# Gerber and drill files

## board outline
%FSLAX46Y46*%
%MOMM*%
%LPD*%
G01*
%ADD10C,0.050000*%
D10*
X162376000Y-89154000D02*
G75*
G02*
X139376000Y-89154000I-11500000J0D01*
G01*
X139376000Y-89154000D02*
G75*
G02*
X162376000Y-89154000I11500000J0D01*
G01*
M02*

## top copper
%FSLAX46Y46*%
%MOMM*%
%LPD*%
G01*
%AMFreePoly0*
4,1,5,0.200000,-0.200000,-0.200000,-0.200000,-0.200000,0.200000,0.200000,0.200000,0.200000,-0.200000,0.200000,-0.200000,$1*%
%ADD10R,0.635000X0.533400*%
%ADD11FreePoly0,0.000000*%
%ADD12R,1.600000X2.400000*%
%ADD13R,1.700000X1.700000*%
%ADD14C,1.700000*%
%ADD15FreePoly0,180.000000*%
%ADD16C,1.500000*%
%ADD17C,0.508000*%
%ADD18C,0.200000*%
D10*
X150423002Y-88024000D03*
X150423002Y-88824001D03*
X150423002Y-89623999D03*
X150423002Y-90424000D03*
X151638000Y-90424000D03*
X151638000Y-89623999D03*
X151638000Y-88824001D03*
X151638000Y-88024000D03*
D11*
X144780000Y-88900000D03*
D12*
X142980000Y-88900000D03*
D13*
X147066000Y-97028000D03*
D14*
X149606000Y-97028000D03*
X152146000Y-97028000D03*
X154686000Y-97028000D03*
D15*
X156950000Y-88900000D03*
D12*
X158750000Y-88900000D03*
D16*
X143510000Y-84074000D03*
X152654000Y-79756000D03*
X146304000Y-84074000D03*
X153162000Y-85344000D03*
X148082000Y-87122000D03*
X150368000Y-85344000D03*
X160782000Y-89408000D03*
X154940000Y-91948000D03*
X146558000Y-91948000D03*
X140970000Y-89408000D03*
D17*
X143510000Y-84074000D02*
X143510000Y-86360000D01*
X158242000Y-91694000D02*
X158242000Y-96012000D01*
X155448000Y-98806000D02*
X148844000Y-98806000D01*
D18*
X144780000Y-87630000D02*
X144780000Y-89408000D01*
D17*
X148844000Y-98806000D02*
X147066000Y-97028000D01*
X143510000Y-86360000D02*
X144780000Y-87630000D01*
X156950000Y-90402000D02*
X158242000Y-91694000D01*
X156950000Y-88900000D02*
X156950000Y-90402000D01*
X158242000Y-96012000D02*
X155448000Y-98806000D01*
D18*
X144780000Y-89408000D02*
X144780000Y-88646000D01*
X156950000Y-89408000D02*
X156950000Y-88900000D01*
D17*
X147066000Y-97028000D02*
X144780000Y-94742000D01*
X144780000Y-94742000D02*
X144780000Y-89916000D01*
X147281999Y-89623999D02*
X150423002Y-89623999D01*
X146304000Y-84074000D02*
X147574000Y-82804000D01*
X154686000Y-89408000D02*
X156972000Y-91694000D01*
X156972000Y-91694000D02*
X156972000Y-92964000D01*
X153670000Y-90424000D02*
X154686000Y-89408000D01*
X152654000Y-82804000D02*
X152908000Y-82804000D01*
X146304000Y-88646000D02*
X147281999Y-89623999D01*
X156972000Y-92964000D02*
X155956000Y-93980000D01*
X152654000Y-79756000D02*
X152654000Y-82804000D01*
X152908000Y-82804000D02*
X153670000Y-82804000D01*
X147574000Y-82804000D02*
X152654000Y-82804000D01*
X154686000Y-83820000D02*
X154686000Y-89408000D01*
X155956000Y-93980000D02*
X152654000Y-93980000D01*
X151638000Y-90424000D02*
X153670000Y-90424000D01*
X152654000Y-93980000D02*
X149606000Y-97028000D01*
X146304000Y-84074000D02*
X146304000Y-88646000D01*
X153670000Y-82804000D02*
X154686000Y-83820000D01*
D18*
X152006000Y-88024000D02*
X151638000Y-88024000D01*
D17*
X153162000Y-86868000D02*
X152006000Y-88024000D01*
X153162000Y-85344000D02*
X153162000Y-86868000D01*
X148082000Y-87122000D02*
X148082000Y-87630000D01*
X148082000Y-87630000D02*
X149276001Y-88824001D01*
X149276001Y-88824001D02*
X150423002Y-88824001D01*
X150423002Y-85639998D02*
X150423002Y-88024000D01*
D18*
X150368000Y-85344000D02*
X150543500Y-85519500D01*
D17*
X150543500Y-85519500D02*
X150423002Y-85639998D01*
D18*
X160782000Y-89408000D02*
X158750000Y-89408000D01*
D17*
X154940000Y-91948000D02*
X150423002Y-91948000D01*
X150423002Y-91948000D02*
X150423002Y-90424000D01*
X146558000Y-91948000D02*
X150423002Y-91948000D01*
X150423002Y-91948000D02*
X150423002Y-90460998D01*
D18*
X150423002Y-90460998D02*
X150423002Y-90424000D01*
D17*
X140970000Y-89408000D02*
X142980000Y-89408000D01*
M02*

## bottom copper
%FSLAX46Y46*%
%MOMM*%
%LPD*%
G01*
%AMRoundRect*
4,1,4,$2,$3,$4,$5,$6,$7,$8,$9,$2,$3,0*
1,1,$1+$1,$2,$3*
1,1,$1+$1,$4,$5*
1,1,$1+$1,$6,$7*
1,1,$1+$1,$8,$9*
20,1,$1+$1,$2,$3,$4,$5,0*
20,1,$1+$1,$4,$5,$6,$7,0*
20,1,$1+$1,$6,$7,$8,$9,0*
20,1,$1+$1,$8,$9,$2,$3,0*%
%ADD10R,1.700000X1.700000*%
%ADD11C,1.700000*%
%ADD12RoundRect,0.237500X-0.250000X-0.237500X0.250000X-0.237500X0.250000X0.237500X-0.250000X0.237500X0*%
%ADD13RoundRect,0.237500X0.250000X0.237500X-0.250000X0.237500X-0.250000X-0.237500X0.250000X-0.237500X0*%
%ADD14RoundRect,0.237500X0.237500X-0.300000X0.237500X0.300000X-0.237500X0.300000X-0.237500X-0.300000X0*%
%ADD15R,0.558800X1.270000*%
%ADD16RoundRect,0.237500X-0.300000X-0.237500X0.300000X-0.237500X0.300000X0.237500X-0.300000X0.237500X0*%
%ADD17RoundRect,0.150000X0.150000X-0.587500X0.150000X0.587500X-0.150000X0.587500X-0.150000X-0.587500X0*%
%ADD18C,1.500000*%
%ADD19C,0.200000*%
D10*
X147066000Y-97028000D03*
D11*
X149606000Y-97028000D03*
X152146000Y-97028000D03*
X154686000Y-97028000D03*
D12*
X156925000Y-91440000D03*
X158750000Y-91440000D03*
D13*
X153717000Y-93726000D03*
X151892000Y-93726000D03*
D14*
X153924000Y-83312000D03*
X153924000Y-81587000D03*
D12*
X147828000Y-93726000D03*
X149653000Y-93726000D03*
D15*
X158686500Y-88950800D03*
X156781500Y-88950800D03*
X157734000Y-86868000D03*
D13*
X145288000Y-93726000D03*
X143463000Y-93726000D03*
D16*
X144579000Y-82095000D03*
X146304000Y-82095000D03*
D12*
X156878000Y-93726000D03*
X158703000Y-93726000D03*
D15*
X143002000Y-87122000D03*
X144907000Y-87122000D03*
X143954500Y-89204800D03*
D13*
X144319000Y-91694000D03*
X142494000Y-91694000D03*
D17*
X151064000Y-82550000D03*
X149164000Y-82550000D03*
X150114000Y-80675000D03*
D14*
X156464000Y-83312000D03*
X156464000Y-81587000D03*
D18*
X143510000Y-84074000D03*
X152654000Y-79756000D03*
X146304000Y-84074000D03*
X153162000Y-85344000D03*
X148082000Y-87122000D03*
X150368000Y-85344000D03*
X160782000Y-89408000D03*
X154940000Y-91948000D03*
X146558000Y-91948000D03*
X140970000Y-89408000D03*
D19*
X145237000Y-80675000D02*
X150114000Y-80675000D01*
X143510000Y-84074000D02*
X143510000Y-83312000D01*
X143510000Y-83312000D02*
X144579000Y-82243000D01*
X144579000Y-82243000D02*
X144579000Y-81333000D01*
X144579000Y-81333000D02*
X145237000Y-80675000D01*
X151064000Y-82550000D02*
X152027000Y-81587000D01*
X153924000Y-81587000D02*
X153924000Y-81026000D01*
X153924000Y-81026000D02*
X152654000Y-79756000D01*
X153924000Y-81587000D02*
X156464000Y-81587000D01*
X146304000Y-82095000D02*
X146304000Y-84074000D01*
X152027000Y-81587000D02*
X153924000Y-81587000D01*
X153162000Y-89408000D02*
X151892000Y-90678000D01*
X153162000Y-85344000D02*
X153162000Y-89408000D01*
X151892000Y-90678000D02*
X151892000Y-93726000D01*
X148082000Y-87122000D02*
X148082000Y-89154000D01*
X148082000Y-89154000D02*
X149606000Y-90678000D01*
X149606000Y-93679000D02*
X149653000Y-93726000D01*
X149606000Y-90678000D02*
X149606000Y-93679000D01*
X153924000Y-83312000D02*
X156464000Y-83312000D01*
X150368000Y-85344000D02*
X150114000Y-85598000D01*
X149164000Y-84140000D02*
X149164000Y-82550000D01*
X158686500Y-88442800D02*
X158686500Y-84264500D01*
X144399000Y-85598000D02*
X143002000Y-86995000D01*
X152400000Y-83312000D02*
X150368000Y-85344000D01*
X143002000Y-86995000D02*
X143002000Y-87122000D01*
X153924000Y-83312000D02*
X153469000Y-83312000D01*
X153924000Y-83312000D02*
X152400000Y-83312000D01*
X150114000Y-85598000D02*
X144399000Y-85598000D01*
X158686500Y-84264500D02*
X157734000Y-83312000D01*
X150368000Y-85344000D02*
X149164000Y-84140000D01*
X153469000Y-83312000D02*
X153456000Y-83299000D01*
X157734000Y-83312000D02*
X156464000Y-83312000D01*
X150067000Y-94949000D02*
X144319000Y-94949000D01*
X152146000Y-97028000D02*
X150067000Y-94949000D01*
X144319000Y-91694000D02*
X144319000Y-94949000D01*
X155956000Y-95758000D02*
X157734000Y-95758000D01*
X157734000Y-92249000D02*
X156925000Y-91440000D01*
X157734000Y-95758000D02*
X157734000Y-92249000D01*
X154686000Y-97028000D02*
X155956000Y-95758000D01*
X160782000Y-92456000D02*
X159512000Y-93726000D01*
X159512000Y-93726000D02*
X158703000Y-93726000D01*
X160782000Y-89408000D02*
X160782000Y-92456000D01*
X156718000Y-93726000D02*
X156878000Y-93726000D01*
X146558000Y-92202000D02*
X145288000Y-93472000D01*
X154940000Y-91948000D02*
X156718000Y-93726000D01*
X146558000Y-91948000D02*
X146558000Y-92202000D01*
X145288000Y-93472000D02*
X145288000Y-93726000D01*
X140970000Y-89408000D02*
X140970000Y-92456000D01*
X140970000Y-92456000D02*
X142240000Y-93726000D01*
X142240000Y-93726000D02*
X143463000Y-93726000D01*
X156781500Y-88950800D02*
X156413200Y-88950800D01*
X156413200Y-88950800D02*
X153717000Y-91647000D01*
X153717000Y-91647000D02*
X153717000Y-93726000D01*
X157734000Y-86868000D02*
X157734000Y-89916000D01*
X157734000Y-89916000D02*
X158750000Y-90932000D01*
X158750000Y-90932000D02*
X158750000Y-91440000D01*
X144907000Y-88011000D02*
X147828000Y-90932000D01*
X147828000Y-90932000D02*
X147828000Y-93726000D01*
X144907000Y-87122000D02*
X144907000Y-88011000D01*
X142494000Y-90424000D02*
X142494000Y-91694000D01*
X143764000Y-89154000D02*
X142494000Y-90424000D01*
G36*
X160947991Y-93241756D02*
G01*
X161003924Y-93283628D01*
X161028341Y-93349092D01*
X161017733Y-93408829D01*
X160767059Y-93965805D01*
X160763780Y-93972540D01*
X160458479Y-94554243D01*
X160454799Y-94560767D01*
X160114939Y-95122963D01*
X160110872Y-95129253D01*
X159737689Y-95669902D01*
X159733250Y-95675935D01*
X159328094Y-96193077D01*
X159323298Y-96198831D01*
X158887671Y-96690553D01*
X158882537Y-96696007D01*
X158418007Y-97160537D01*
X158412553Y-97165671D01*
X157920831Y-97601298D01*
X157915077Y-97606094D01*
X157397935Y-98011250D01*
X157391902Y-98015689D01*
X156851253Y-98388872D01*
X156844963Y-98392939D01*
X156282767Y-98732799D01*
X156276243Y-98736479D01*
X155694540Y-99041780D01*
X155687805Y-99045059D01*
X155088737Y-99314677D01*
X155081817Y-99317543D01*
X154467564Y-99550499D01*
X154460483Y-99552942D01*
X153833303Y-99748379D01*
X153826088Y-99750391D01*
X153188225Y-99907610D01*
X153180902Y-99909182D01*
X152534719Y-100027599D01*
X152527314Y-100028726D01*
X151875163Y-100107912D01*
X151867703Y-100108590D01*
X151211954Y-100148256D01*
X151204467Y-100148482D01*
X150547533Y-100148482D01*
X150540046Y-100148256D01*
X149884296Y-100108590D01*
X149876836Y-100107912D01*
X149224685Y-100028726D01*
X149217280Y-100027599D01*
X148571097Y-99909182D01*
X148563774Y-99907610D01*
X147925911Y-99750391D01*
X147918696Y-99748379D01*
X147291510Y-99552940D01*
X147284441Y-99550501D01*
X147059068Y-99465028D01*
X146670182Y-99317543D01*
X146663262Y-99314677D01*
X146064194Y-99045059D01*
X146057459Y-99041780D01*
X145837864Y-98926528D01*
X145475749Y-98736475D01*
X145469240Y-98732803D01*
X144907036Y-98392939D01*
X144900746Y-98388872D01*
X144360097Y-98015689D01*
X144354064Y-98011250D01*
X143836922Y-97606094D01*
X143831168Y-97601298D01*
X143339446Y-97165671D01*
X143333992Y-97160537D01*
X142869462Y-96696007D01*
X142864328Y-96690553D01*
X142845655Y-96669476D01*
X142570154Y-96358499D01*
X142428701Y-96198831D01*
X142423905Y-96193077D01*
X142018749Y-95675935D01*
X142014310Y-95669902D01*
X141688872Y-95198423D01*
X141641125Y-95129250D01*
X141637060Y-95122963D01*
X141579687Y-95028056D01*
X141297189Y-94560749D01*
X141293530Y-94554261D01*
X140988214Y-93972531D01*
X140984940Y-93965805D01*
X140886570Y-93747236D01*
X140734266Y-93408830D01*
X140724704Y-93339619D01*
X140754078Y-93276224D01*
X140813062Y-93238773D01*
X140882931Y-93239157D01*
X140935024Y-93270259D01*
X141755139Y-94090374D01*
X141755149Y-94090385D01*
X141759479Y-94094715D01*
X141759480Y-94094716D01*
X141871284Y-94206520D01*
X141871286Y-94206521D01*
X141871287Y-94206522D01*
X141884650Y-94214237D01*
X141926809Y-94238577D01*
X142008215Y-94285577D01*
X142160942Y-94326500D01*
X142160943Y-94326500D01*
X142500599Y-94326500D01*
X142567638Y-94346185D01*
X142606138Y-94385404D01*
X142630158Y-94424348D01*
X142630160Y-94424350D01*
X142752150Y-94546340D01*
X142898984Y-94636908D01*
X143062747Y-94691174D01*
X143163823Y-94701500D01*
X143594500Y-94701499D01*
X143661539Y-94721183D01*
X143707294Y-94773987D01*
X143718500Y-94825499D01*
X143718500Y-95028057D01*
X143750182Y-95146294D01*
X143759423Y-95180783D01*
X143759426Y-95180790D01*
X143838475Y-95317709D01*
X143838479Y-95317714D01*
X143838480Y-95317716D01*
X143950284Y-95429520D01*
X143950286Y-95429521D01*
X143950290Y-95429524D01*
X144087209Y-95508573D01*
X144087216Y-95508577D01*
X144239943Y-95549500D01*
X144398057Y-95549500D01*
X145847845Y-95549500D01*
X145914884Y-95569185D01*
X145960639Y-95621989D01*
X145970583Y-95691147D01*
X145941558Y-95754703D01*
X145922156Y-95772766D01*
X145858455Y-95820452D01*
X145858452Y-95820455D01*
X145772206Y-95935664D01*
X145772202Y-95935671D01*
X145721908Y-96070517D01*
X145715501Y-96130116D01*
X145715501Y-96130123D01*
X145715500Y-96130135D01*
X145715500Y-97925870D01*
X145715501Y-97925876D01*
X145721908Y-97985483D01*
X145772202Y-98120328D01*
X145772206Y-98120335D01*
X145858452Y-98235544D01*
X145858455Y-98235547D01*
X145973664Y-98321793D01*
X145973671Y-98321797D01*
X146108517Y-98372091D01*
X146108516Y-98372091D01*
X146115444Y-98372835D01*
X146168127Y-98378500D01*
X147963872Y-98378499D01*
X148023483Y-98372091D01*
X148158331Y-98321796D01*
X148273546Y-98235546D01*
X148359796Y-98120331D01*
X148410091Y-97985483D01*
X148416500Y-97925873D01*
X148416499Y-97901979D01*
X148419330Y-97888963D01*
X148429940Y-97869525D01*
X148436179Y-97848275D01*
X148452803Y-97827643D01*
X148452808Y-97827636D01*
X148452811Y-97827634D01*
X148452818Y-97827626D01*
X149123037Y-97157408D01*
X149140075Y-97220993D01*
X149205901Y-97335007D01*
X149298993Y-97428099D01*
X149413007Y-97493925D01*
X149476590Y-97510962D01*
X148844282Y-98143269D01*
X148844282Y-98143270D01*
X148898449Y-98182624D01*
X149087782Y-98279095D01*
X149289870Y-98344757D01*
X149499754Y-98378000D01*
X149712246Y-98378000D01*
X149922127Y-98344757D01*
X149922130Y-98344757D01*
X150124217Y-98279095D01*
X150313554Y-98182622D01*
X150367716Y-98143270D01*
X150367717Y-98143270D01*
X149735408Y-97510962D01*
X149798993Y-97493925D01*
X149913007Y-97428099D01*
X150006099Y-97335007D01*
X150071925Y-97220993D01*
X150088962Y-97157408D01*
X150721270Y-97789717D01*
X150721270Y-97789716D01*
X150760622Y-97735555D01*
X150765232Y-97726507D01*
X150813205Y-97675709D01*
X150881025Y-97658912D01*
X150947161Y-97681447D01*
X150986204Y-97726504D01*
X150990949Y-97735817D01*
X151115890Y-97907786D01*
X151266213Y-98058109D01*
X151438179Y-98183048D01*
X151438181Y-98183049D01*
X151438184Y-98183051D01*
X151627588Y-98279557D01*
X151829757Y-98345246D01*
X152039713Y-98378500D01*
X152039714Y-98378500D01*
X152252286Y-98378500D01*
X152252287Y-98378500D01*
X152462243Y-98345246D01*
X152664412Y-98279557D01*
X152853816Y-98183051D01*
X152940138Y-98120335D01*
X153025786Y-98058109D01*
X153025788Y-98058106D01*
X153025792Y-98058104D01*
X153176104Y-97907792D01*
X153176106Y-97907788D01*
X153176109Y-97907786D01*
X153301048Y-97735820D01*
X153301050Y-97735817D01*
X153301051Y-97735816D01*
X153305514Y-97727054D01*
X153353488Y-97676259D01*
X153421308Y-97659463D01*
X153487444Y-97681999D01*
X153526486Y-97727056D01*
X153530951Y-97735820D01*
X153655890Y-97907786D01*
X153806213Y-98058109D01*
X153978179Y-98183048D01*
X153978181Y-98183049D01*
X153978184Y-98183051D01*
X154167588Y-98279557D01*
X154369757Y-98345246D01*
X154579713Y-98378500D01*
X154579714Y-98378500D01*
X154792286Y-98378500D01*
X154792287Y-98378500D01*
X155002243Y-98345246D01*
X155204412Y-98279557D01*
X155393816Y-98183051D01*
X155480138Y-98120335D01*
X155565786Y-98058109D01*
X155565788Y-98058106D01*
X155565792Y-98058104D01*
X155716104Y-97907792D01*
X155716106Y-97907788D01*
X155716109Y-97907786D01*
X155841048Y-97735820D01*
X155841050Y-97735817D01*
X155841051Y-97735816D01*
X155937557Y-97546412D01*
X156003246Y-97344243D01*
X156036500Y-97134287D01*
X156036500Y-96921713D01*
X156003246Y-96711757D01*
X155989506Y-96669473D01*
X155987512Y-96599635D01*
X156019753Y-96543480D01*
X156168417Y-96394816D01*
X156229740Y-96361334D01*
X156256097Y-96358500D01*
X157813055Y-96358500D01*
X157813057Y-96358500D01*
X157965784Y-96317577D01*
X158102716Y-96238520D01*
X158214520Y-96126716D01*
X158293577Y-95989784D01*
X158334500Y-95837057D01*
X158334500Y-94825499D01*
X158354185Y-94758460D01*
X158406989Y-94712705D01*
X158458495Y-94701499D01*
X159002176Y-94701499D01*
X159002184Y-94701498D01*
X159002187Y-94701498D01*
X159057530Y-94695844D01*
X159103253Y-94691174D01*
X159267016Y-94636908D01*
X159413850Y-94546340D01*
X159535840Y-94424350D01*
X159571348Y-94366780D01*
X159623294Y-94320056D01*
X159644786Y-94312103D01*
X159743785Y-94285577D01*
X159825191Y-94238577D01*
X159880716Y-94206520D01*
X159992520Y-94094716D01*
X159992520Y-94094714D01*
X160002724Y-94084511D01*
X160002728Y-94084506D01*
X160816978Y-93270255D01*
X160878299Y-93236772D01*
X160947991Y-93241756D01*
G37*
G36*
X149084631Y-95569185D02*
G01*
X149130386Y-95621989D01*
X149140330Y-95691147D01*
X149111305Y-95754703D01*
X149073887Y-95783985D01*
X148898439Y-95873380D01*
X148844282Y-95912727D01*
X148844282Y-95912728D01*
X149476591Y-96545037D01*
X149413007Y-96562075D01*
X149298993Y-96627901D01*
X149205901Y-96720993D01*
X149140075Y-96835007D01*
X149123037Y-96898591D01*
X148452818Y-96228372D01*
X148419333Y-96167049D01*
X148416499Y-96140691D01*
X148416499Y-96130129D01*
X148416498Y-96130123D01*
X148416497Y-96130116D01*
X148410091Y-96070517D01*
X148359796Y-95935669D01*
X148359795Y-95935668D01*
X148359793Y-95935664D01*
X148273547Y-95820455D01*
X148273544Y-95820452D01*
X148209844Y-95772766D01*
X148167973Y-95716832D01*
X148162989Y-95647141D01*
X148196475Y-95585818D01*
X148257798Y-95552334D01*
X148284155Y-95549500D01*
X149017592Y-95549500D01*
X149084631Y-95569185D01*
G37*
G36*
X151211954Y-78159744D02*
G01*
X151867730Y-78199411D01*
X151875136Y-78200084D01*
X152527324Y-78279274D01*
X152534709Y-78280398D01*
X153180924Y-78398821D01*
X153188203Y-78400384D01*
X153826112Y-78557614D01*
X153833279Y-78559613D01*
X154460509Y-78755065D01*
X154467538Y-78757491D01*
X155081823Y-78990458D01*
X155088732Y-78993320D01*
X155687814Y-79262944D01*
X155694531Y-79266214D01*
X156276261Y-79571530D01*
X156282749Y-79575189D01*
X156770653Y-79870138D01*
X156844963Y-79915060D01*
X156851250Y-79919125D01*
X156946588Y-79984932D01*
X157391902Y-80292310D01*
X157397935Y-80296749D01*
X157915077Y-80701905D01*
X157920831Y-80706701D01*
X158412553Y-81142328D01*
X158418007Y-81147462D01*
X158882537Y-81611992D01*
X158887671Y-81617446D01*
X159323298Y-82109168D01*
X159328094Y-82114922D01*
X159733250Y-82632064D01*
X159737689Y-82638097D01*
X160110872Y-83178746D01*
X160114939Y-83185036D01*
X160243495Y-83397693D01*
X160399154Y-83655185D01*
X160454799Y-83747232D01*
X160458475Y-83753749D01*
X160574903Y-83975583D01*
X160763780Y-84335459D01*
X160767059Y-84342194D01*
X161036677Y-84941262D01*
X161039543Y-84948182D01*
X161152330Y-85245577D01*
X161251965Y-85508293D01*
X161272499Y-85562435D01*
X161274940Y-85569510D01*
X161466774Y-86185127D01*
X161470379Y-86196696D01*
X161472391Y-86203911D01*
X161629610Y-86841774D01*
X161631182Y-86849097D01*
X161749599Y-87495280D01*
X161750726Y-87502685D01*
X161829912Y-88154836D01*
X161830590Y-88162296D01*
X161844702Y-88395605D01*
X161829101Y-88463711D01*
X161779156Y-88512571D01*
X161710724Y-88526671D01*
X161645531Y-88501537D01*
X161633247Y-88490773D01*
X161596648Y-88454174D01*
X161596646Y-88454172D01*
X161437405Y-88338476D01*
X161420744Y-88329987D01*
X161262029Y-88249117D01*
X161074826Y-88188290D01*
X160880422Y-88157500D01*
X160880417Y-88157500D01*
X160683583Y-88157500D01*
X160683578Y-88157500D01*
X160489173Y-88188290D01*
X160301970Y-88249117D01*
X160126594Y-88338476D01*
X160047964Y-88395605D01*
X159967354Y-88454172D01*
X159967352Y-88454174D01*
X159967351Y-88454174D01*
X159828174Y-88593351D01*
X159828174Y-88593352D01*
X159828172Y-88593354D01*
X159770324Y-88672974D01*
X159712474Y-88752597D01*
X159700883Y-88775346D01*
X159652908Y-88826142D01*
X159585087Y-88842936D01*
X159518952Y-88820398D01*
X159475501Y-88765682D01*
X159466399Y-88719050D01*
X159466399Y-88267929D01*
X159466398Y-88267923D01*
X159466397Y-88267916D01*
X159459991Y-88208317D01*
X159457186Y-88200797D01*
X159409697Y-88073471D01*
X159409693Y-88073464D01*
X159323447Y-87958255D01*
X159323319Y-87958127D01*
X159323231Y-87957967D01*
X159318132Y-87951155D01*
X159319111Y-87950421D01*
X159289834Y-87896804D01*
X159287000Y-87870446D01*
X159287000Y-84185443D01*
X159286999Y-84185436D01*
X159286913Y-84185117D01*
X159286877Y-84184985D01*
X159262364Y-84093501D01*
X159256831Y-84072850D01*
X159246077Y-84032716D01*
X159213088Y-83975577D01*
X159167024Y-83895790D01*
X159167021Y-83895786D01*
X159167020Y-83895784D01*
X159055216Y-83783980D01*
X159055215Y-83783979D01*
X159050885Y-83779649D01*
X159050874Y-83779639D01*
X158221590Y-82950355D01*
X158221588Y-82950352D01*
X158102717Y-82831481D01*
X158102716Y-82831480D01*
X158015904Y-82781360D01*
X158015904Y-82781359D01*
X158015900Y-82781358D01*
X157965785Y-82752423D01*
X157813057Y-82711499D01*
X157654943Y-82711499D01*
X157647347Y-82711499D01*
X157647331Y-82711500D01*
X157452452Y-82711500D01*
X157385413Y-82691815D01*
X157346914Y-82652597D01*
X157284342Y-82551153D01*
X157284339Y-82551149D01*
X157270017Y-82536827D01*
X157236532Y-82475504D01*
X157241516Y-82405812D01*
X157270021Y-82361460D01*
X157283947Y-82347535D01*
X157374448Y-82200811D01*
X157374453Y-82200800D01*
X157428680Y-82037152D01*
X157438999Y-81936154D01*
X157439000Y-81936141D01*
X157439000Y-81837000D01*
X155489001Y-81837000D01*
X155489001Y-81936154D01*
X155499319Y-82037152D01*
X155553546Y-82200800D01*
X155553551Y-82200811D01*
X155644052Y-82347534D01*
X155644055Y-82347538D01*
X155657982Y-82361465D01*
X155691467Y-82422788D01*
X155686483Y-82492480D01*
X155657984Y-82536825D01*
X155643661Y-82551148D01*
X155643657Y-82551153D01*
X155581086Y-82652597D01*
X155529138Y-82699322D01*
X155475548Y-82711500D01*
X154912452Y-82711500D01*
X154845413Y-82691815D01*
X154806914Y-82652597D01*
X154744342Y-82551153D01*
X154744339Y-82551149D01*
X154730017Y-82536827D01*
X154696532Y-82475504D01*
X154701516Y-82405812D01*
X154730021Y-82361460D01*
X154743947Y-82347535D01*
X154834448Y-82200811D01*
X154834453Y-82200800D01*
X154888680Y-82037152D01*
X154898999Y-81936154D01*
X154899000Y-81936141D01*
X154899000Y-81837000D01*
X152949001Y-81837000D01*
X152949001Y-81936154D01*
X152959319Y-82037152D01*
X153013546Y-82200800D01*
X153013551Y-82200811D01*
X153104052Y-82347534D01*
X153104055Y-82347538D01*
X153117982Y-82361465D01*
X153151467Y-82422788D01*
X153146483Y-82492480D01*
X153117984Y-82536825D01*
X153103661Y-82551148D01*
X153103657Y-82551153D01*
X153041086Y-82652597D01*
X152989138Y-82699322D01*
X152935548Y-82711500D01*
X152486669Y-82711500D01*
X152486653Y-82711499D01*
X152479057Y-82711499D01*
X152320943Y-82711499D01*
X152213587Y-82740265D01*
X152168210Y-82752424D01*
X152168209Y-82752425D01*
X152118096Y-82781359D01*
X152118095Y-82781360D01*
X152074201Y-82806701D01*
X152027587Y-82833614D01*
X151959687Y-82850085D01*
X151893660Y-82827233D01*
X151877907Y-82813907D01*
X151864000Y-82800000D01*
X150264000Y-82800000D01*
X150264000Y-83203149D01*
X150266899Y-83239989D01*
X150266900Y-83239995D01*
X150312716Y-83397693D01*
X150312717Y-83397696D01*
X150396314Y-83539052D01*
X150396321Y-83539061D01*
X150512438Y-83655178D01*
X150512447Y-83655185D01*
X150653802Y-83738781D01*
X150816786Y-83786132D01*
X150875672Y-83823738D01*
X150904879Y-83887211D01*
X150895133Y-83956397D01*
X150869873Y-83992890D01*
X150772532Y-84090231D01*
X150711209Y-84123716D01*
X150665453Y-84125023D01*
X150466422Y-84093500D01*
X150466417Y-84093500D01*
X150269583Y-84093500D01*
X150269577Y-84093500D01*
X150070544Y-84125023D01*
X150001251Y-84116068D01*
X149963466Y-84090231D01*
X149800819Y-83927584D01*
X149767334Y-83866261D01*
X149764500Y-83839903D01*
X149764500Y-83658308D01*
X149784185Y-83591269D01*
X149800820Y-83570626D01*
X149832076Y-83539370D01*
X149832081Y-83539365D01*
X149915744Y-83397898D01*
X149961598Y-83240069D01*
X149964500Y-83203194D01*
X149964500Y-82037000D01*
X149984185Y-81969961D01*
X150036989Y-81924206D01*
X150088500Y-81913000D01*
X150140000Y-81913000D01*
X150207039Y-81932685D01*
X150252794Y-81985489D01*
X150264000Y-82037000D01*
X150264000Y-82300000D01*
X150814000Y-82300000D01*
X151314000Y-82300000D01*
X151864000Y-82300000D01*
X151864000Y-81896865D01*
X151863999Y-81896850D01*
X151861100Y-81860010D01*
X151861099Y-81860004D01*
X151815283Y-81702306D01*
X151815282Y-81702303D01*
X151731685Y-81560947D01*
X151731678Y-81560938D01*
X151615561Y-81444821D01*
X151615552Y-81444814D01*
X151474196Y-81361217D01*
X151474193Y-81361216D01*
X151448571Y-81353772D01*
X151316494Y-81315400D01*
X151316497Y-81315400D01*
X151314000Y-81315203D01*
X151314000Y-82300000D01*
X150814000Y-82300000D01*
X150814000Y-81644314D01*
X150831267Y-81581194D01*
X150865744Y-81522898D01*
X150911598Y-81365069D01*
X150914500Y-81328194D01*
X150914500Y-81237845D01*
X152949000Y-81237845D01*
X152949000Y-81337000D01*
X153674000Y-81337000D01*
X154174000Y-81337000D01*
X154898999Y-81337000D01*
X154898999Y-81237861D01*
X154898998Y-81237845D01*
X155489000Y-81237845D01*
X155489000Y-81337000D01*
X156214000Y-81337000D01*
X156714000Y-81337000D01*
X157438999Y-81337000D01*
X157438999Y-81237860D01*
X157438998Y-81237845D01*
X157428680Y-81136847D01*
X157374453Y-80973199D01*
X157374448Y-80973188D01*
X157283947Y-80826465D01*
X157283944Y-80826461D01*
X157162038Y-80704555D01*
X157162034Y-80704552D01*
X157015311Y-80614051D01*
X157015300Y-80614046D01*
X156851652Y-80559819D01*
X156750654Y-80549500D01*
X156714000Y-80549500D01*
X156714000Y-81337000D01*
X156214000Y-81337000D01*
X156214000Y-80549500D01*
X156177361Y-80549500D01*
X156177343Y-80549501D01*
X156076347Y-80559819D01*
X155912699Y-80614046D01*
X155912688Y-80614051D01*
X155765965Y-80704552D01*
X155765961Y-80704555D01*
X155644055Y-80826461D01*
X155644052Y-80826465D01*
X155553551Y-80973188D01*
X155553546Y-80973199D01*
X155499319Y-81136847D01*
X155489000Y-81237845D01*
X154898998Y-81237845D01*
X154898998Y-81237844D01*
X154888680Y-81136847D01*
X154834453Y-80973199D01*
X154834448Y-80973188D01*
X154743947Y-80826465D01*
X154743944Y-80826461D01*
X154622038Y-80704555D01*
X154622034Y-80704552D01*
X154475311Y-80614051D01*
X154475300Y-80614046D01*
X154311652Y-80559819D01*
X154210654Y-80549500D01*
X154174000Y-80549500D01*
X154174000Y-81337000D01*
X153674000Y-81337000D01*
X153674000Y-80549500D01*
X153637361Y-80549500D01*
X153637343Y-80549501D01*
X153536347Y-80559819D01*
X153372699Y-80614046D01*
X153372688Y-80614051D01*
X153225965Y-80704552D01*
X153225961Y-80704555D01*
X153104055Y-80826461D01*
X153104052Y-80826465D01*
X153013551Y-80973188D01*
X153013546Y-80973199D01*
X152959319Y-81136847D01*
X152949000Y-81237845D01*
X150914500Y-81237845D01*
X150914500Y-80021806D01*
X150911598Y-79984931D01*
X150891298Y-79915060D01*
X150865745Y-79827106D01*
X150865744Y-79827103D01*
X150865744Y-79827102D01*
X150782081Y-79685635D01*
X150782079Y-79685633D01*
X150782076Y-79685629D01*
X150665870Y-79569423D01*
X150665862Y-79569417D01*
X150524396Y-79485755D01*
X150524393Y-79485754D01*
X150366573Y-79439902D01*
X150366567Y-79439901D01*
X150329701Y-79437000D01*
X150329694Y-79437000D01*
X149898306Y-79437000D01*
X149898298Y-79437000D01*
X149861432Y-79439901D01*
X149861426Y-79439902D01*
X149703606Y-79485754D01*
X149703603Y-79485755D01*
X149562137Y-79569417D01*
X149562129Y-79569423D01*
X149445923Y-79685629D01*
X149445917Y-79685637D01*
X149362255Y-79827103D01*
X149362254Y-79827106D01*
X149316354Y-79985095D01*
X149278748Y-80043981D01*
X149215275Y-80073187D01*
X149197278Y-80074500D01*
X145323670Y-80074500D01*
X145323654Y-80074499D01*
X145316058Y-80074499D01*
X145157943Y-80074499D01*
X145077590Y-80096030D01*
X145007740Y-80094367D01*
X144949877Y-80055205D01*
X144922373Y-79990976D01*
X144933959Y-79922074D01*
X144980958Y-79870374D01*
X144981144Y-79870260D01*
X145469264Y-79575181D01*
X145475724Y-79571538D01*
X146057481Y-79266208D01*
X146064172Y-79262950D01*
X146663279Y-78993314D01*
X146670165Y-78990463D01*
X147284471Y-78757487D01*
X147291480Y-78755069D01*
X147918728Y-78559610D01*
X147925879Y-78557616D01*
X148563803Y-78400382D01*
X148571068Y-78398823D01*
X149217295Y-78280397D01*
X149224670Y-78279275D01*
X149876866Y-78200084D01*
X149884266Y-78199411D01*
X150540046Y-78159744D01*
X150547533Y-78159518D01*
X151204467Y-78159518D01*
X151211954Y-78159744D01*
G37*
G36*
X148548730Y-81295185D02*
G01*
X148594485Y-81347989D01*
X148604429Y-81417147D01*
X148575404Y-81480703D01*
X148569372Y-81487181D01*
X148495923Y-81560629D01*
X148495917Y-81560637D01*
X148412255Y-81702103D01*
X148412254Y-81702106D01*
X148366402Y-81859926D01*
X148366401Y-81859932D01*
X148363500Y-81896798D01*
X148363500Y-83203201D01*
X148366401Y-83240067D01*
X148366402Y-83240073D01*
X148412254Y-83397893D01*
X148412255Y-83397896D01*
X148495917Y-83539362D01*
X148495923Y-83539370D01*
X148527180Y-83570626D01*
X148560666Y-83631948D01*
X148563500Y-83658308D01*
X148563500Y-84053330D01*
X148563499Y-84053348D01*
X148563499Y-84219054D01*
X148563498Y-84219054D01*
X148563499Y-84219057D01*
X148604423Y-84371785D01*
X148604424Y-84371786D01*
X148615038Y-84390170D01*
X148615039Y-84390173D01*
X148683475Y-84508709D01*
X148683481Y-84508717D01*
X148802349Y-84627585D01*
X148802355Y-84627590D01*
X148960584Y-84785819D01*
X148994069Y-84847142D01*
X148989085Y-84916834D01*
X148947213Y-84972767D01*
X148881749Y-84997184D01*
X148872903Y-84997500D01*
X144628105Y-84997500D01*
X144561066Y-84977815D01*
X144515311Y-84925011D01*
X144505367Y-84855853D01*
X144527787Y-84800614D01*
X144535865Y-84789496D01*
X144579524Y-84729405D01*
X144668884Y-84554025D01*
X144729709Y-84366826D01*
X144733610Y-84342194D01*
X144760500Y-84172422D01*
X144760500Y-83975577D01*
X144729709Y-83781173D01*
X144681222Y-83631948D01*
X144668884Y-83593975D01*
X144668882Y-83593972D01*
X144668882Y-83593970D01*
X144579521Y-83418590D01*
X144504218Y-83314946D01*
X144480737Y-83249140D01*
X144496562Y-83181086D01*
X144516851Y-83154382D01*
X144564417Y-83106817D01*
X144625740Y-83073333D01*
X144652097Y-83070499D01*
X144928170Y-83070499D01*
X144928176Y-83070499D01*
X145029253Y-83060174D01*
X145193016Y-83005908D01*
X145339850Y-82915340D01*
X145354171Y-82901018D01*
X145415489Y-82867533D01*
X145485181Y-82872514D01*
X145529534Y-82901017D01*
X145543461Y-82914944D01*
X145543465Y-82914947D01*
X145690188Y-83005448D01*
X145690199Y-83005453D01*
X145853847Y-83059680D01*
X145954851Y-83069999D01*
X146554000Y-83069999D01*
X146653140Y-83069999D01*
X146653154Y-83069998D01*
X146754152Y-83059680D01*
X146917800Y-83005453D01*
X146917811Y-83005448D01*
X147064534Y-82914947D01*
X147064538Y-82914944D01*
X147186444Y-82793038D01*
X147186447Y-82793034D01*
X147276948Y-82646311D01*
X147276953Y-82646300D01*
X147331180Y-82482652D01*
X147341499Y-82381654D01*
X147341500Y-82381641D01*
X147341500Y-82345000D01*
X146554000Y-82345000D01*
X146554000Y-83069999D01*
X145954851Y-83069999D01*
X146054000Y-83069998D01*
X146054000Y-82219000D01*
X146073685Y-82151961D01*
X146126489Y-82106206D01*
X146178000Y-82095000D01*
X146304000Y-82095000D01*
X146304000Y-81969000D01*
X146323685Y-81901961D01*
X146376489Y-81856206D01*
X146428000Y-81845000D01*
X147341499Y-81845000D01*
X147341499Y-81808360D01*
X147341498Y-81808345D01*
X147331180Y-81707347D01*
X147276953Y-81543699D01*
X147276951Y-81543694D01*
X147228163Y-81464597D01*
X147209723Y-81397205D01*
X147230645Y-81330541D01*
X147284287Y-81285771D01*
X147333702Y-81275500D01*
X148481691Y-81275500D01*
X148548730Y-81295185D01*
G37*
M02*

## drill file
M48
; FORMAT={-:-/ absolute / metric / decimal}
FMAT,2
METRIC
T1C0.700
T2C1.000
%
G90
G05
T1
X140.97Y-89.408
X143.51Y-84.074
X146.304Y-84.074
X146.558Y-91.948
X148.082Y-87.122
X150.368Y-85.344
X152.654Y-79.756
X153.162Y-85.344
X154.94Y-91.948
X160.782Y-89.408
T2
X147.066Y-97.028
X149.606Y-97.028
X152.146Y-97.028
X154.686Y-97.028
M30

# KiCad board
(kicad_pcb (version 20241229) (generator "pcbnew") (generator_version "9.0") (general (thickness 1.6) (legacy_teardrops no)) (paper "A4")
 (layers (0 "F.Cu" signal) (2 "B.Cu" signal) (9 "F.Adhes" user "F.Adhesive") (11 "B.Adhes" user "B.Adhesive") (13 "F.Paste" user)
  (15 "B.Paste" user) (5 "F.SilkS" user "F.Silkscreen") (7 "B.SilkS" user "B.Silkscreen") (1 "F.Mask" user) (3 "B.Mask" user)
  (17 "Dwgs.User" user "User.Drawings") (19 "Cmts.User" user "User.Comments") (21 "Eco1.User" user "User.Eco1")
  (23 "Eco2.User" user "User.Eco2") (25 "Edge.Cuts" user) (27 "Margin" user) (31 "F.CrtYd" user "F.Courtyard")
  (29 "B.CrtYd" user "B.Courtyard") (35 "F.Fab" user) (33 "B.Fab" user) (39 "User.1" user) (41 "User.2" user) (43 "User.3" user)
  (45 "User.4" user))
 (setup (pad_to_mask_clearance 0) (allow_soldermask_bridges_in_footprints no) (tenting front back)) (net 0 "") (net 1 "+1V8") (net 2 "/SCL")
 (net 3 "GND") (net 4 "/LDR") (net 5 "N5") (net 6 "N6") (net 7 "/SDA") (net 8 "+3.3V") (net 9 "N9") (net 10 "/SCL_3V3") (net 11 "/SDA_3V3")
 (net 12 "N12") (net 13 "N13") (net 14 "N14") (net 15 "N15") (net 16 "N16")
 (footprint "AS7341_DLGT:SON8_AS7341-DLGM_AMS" (layer "F.Cu") (at 151.030501 89.224)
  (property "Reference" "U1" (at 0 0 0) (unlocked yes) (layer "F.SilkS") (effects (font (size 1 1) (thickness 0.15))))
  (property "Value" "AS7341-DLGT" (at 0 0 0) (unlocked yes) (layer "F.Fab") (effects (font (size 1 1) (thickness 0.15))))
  (pad "1" smd rect (at -0.607499 -1.2) (size 0.635 0.5334) (layers "F.Cu" "F.Mask" "F.Paste") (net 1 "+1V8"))
  (pad "2" smd rect (at -0.607499 -0.399999) (size 0.635 0.5334) (layers "F.Cu" "F.Mask" "F.Paste") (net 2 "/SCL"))
  (pad "3" smd rect (at -0.607499 0.399999) (size 0.635 0.5334) (layers "F.Cu" "F.Mask" "F.Paste") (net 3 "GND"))
  (pad "4" smd rect (at -0.607499 1.2) (size 0.635 0.5334) (layers "F.Cu" "F.Mask" "F.Paste") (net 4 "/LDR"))
  (pad "5" smd rect (at 0.607499 1.2) (size 0.635 0.5334) (layers "F.Cu" "F.Mask" "F.Paste") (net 3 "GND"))
  (pad "6" smd rect (at 0.607499 0.399999) (size 0.635 0.5334) (layers "F.Cu" "F.Mask" "F.Paste") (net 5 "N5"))
  (pad "7" smd rect (at 0.607499 -0.399999) (size 0.635 0.5334) (layers "F.Cu" "F.Mask" "F.Paste") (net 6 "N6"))
  (pad "8" smd rect (at 0.607499 -1.2) (size 0.635 0.5334) (layers "F.Cu" "F.Mask" "F.Paste") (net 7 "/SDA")))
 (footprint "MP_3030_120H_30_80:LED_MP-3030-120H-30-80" (layer "F.Cu") (at 143.78 88.9)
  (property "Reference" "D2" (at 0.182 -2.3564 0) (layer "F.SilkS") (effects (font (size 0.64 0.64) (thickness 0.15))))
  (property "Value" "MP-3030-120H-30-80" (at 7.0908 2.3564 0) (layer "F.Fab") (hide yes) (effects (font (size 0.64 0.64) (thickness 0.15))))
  (pad "A" smd custom (at 1 0) (size 0.4 0.4) (layers "F.Cu") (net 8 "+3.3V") (options (clearance outline) (anchor rect)) (primitives))
  (pad "C" smd rect (at -0.8 0) (size 1.6 2.4) (layers "F.Cu" "F.Mask" "F.Paste") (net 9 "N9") (solder_mask_margin 0.102)))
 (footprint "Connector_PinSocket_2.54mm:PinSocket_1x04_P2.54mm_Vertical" (layer "F.Cu") (at 147.066 97.028 90)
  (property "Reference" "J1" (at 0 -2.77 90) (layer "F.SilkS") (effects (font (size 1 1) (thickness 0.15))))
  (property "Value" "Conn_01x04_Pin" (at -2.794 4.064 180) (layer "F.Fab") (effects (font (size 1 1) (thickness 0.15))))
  (pad "1" thru_hole rect (at 0 0 90) (size 1.7 1.7) (drill 1) (layers "*.Cu" "*.Mask") (remove_unused_layers no) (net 8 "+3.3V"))
  (pad "2" thru_hole circle (at 0 2.54 90) (size 1.7 1.7) (drill 1) (layers "*.Cu" "*.Mask") (remove_unused_layers no) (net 3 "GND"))
  (pad "3" thru_hole circle (at 0 5.08 90) (size 1.7 1.7) (drill 1) (layers "*.Cu" "*.Mask") (remove_unused_layers no) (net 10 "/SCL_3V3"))
  (pad "4" thru_hole circle (at 0 7.62 90) (size 1.7 1.7) (drill 1) (layers "*.Cu" "*.Mask") (remove_unused_layers no) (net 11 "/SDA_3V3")))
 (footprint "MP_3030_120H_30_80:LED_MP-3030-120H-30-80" (layer "F.Cu") (at 157.95 88.9 180)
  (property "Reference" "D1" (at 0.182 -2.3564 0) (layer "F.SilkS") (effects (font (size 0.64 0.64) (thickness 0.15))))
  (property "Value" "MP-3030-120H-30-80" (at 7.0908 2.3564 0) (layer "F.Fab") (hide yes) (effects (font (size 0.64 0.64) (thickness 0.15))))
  (pad "A" smd custom (at 1 0 180) (size 0.4 0.4) (layers "F.Cu") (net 8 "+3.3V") (options (clearance outline) (anchor rect)) (primitives))
  (pad "C" smd rect (at -0.8 0 180) (size 1.6 2.4) (layers "F.Cu" "F.Mask" "F.Paste") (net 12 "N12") (solder_mask_margin 0.102)))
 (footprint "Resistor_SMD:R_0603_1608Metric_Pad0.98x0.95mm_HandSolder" (layer "B.Cu") (at 157.8375 91.44)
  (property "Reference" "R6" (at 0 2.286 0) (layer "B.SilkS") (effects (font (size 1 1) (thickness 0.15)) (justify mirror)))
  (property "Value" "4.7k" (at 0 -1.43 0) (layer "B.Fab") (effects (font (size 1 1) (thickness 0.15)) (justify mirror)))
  (pad "1" smd roundrect (at -0.9125 0) (size 0.975 0.95) (layers "B.Cu" "B.Mask" "B.Paste") (roundrect_rratio 0.25) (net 11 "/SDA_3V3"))
  (pad "2" smd roundrect (at 0.9125 0) (size 0.975 0.95) (layers "B.Cu" "B.Mask" "B.Paste") (roundrect_rratio 0.25) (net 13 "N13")))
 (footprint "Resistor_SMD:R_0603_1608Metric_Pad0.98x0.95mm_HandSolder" (layer "B.Cu") (at 152.8045 93.726 180)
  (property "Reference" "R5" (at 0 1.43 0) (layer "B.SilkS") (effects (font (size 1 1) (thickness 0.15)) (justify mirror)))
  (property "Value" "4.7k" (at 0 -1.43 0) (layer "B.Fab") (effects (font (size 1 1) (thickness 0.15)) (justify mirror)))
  (pad "1" smd roundrect (at -0.9125 0 180) (size 0.975 0.95) (layers "B.Cu" "B.Mask" "B.Paste") (roundrect_rratio 0.25) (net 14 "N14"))
  (pad "2" smd roundrect (at 0.9125 0 180) (size 0.975 0.95) (layers "B.Cu" "B.Mask" "B.Paste") (roundrect_rratio 0.25) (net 7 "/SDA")))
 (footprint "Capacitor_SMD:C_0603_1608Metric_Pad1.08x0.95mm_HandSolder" (layer "B.Cu") (at 153.924 82.4495 90)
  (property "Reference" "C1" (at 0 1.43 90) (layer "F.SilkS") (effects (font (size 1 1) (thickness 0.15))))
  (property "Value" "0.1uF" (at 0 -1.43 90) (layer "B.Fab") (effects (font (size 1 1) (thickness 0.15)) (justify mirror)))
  (pad "1" smd roundrect (at -0.8625 0 90) (size 1.075 0.95) (layers "B.Cu" "B.Mask" "B.Paste") (roundrect_rratio 0.25) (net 1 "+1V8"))
  (pad "2" smd roundrect (at 0.8625 0 90) (size 1.075 0.95) (layers "B.Cu" "B.Mask" "B.Paste") (roundrect_rratio 0.25) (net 3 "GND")))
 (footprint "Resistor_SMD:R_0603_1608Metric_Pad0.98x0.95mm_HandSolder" (layer "B.Cu") (at 148.7405 93.726)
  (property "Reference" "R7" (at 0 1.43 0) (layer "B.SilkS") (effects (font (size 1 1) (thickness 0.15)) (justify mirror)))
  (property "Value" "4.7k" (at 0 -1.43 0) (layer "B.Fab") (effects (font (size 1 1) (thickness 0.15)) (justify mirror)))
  (pad "1" smd roundrect (at -0.9125 0) (size 0.975 0.95) (layers "B.Cu" "B.Mask" "B.Paste") (roundrect_rratio 0.25) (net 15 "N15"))
  (pad "2" smd roundrect (at 0.9125 0) (size 0.975 0.95) (layers "B.Cu" "B.Mask" "B.Paste") (roundrect_rratio 0.25) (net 2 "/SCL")))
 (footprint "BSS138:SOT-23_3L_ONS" (layer "B.Cu") (at 157.734 87.9094 180)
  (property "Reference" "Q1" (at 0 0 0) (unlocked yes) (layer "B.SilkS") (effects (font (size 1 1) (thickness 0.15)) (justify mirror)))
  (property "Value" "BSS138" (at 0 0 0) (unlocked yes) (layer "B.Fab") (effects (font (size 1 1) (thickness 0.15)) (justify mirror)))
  (pad "1" smd rect (at -0.9525 -1.0414 180) (size 0.5588 1.27) (layers "B.Cu" "B.Mask" "B.Paste") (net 1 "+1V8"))
  (pad "2" smd rect (at 0.9525 -1.0414 180) (size 0.5588 1.27) (layers "B.Cu" "B.Mask" "B.Paste") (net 14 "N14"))
  (pad "3" smd rect (at 0 1.0414 180) (size 0.5588 1.27) (layers "B.Cu" "B.Mask" "B.Paste") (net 13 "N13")))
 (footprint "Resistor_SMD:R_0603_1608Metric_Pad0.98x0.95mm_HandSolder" (layer "B.Cu") (at 144.3755 93.726 180)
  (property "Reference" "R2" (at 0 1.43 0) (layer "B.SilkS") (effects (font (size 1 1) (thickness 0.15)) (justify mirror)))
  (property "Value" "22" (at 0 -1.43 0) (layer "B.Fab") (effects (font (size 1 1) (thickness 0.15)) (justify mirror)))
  (pad "1" smd roundrect (at -0.9125 0 180) (size 0.975 0.95) (layers "B.Cu" "B.Mask" "B.Paste") (roundrect_rratio 0.25) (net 4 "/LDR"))
  (pad "2" smd roundrect (at 0.9125 0 180) (size 0.975 0.95) (layers "B.Cu" "B.Mask" "B.Paste") (roundrect_rratio 0.25) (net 9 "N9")))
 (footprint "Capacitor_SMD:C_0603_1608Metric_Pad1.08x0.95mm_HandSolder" (layer "B.Cu") (at 145.4415 82.095)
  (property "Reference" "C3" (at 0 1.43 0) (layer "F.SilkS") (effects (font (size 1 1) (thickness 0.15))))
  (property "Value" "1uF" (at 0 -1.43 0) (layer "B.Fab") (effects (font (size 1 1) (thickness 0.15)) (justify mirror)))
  (pad "1" smd roundrect (at -0.8625 0) (size 1.075 0.95) (layers "B.Cu" "B.Mask" "B.Paste") (roundrect_rratio 0.25) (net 8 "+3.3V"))
  (pad "2" smd roundrect (at 0.8625 0) (size 1.075 0.95) (layers "B.Cu" "B.Mask" "B.Paste") (roundrect_rratio 0.25) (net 3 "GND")))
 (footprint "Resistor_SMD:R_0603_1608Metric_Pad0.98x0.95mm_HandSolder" (layer "B.Cu") (at 157.7905 93.726)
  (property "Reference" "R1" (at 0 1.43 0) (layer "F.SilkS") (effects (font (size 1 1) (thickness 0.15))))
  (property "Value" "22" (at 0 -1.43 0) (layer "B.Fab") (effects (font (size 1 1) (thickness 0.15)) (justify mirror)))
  (pad "1" smd roundrect (at -0.9125 0) (size 0.975 0.95) (layers "B.Cu" "B.Mask" "B.Paste") (roundrect_rratio 0.25) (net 4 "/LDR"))
  (pad "2" smd roundrect (at 0.9125 0) (size 0.975 0.95) (layers "B.Cu" "B.Mask" "B.Paste") (roundrect_rratio 0.25) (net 12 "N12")))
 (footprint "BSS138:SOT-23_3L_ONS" (layer "B.Cu") (at 143.9545 88.1634)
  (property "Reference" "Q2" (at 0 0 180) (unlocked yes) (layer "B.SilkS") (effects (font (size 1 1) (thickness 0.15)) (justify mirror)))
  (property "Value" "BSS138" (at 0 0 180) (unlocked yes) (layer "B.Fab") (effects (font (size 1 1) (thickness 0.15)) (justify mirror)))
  (pad "1" smd rect (at -0.9525 -1.0414) (size 0.5588 1.27) (layers "B.Cu" "B.Mask" "B.Paste") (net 1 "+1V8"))
  (pad "2" smd rect (at 0.9525 -1.0414) (size 0.5588 1.27) (layers "B.Cu" "B.Mask" "B.Paste") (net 15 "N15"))
  (pad "3" smd rect (at 0 1.0414) (size 0.5588 1.27) (layers "B.Cu" "B.Mask" "B.Paste") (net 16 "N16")))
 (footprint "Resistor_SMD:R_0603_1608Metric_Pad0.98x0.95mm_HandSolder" (layer "B.Cu") (at 143.4065 91.694 180)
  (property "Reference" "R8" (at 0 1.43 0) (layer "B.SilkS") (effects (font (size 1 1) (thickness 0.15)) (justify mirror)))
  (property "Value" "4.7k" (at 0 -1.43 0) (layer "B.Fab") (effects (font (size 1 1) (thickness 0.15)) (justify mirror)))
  (pad "1" smd roundrect (at -0.9125 0 180) (size 0.975 0.95) (layers "B.Cu" "B.Mask" "B.Paste") (roundrect_rratio 0.25) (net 10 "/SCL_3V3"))
  (pad "2" smd roundrect (at 0.9125 0 180) (size 0.975 0.95) (layers "B.Cu" "B.Mask" "B.Paste") (roundrect_rratio 0.25) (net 16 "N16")))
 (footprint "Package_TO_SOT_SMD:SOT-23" (layer "B.Cu") (at 150.114 81.6125 90)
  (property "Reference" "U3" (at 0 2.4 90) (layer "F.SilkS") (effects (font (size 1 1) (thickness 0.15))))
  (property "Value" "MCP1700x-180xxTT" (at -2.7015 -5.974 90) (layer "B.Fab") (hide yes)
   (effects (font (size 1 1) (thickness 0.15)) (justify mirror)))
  (pad "1" smd roundrect (at -0.9375 0.95 90) (size 1.475 0.6) (layers "B.Cu" "B.Mask" "B.Paste") (roundrect_rratio 0.25) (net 3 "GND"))
  (pad "2" smd roundrect (at -0.9375 -0.95 90) (size 1.475 0.6) (layers "B.Cu" "B.Mask" "B.Paste") (roundrect_rratio 0.25) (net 1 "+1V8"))
  (pad "3" smd roundrect (at 0.9375 0 90) (size 1.475 0.6) (layers "B.Cu" "B.Mask" "B.Paste") (roundrect_rratio 0.25) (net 8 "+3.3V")))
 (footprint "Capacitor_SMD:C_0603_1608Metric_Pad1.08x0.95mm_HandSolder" (layer "B.Cu") (at 156.464 82.4495 90)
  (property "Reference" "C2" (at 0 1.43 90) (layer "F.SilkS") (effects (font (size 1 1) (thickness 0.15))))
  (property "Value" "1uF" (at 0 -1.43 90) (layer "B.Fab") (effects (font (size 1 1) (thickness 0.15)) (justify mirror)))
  (pad "1" smd roundrect (at -0.8625 0 90) (size 1.075 0.95) (layers "B.Cu" "B.Mask" "B.Paste") (roundrect_rratio 0.25) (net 1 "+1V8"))
  (pad "2" smd roundrect (at 0.8625 0 90) (size 1.075 0.95) (layers "B.Cu" "B.Mask" "B.Paste") (roundrect_rratio 0.25) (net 3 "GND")))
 (gr_circle (center 150.876 89.154) (end 162.376 89.154) (stroke (width 0.05) (type solid)) (fill no) (layer "Edge.Cuts"))
 (segment (start 143.51 84.074) (end 143.51 86.36) (width 0.508) (layer "F.Cu") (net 8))
 (segment (start 158.242 91.694) (end 158.242 96.012) (width 0.508) (layer "F.Cu") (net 8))
 (segment (start 155.448 98.806) (end 148.844 98.806) (width 0.508) (layer "F.Cu") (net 8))
 (segment (start 144.78 87.63) (end 144.78 89.408) (width 0.2) (layer "F.Cu") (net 8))
 (segment (start 148.844 98.806) (end 147.066 97.028) (width 0.508) (layer "F.Cu") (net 8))
 (segment (start 143.51 86.36) (end 144.78 87.63) (width 0.508) (layer "F.Cu") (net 8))
 (segment (start 156.95 90.402) (end 158.242 91.694) (width 0.508) (layer "F.Cu") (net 8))
 (segment (start 156.95 88.9) (end 156.95 90.402) (width 0.508) (layer "F.Cu") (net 8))
 (segment (start 158.242 96.012) (end 155.448 98.806) (width 0.508) (layer "F.Cu") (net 8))
 (segment (start 144.78 89.408) (end 144.78 88.646) (width 0.2) (layer "F.Cu") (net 8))
 (segment (start 156.95 89.408) (end 156.95 88.9) (width 0.2) (layer "F.Cu") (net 8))
 (segment (start 147.066 97.028) (end 144.78 94.742) (width 0.508) (layer "F.Cu") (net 8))
 (segment (start 144.78 94.742) (end 144.78 89.916) (width 0.508) (layer "F.Cu") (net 8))
 (via (at 143.51 84.074) (size 1.5) (drill 0.7) (layers "F.Cu" "B.Cu") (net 8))
 (segment (start 145.237 80.675) (end 150.114 80.675) (width 0.2) (layer "B.Cu") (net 8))
 (segment (start 143.51 84.074) (end 143.51 83.312) (width 0.2) (layer "B.Cu") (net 8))
 (segment (start 143.51 83.312) (end 144.579 82.243) (width 0.2) (layer "B.Cu") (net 8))
 (segment (start 144.579 82.243) (end 144.579 81.333) (width 0.2) (layer "B.Cu") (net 8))
 (segment (start 144.579 81.333) (end 145.237 80.675) (width 0.2) (layer "B.Cu") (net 8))
 (segment (start 147.281999 89.623999) (end 150.423002 89.623999) (width 0.508) (layer "F.Cu") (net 3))
 (segment (start 146.304 84.074) (end 147.574 82.804) (width 0.508) (layer "F.Cu") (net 3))
 (segment (start 154.686 89.408) (end 156.972 91.694) (width 0.508) (layer "F.Cu") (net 3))
 (segment (start 156.972 91.694) (end 156.972 92.964) (width 0.508) (layer "F.Cu") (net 3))
 (segment (start 153.67 90.424) (end 154.686 89.408) (width 0.508) (layer "F.Cu") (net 3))
 (segment (start 152.654 82.804) (end 152.908 82.804) (width 0.508) (layer "F.Cu") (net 3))
 (segment (start 146.304 88.646) (end 147.281999 89.623999) (width 0.508) (layer "F.Cu") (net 3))
 (segment (start 156.972 92.964) (end 155.956 93.98) (width 0.508) (layer "F.Cu") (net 3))
 (segment (start 152.654 79.756) (end 152.654 82.804) (width 0.508) (layer "F.Cu") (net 3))
 (segment (start 152.908 82.804) (end 153.67 82.804) (width 0.508) (layer "F.Cu") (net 3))
 (segment (start 147.574 82.804) (end 152.654 82.804) (width 0.508) (layer "F.Cu") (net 3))
 (segment (start 154.686 83.82) (end 154.686 89.408) (width 0.508) (layer "F.Cu") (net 3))
 (segment (start 155.956 93.98) (end 152.654 93.98) (width 0.508) (layer "F.Cu") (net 3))
 (segment (start 151.638 90.424) (end 153.67 90.424) (width 0.508) (layer "F.Cu") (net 3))
 (segment (start 152.654 93.98) (end 149.606 97.028) (width 0.508) (layer "F.Cu") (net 3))
 (segment (start 146.304 84.074) (end 146.304 88.646) (width 0.508) (layer "F.Cu") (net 3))
 (segment (start 153.67 82.804) (end 154.686 83.82) (width 0.508) (layer "F.Cu") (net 3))
 (via (at 152.654 79.756) (size 1.5) (drill 0.7) (layers "F.Cu" "B.Cu") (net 3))
 (via (at 146.304 84.074) (size 1.5) (drill 0.7) (layers "F.Cu" "B.Cu") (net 3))
 (segment (start 151.064 82.55) (end 152.027 81.587) (width 0.2) (layer "B.Cu") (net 3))
 (segment (start 153.924 81.587) (end 153.924 81.026) (width 0.2) (layer "B.Cu") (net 3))
 (segment (start 153.924 81.026) (end 152.654 79.756) (width 0.2) (layer "B.Cu") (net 3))
 (segment (start 153.924 81.587) (end 156.464 81.587) (width 0.2) (layer "B.Cu") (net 3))
 (segment (start 146.304 82.095) (end 146.304 84.074) (width 0.2) (layer "B.Cu") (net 3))
 (segment (start 152.027 81.587) (end 153.924 81.587) (width 0.2) (layer "B.Cu") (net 3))
 (segment (start 152.006 88.024) (end 151.638 88.024) (width 0.2) (layer "F.Cu") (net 7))
 (segment (start 153.162 86.868) (end 152.006 88.024) (width 0.508) (layer "F.Cu") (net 7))
 (segment (start 153.162 85.344) (end 153.162 86.868) (width 0.508) (layer "F.Cu") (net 7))
 (via (at 153.162 85.344) (size 1.5) (drill 0.7) (layers "F.Cu" "B.Cu") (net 7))
 (segment (start 153.162 89.408) (end 151.892 90.678) (width 0.2) (layer "B.Cu") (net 7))
 (segment (start 153.162 85.344) (end 153.162 89.408) (width 0.2) (layer "B.Cu") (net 7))
 (segment (start 151.892 90.678) (end 151.892 93.726) (width 0.2) (layer "B.Cu") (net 7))
 (segment (start 148.082 87.122) (end 148.082 87.63) (width 0.508) (layer "F.Cu") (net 2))
 (segment (start 148.082 87.63) (end 149.276001 88.824001) (width 0.508) (layer "F.Cu") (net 2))
 (segment (start 149.276001 88.824001) (end 150.423002 88.824001) (width 0.508) (layer "F.Cu") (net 2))
 (via (at 148.082 87.122) (size 1.5) (drill 0.7) (layers "F.Cu" "B.Cu") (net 2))
 (segment (start 148.082 87.122) (end 148.082 89.154) (width 0.2) (layer "B.Cu") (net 2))
 (segment (start 148.082 89.154) (end 149.606 90.678) (width 0.2) (layer "B.Cu") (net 2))
 (segment (start 149.606 93.679) (end 149.653 93.726) (width 0.2) (layer "B.Cu") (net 2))
 (segment (start 149.606 90.678) (end 149.606 93.679) (width 0.2) (layer "B.Cu") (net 2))
 (segment (start 150.423002 85.639998) (end 150.423002 88.024) (width 0.508) (layer "F.Cu") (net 1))
 (segment (start 150.368 85.344) (end 150.5435 85.5195) (width 0.2) (layer "F.Cu") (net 1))
 (segment (start 150.5435 85.5195) (end 150.423002 85.639998) (width 0.508) (layer "F.Cu") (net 1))
 (via (at 150.368 85.344) (size 1.5) (drill 0.7) (layers "F.Cu" "B.Cu") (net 1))
 (segment (start 153.924 83.312) (end 156.464 83.312) (width 0.2) (layer "B.Cu") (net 1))
 (segment (start 150.368 85.344) (end 150.114 85.598) (width 0.2) (layer "B.Cu") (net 1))
 (segment (start 149.164 84.14) (end 149.164 82.55) (width 0.2) (layer "B.Cu") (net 1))
 (segment (start 158.6865 88.4428) (end 158.6865 84.2645) (width 0.2) (layer "B.Cu") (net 1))
 (segment (start 144.399 85.598) (end 143.002 86.995) (width 0.2) (layer "B.Cu") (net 1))
 (segment (start 152.4 83.312) (end 150.368 85.344) (width 0.2) (layer "B.Cu") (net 1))
 (segment (start 143.002 86.995) (end 143.002 87.122) (width 0.2) (layer "B.Cu") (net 1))
 (segment (start 153.924 83.312) (end 153.469 83.312) (width 0.2) (layer "B.Cu") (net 1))
 (segment (start 153.924 83.312) (end 152.4 83.312) (width 0.2) (layer "B.Cu") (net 1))
 (segment (start 150.114 85.598) (end 144.399 85.598) (width 0.2) (layer "B.Cu") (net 1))
 (segment (start 158.6865 84.2645) (end 157.734 83.312) (width 0.2) (layer "B.Cu") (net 1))
 (segment (start 150.368 85.344) (end 149.164 84.14) (width 0.2) (layer "B.Cu") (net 1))
 (segment (start 153.469 83.312) (end 153.456 83.299) (width 0.2) (layer "B.Cu") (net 1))
 (segment (start 157.734 83.312) (end 156.464 83.312) (width 0.2) (layer "B.Cu") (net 1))
 (segment (start 150.067 94.949) (end 144.319 94.949) (width 0.2) (layer "B.Cu") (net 10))
 (segment (start 152.146 97.028) (end 150.067 94.949) (width 0.2) (layer "B.Cu") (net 10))
 (segment (start 144.319 91.694) (end 144.319 94.949) (width 0.2) (layer "B.Cu") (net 10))
 (segment (start 155.956 95.758) (end 157.734 95.758) (width 0.2) (layer "B.Cu") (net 11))
 (segment (start 157.734 92.249) (end 156.925 91.44) (width 0.2) (layer "B.Cu") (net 11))
 (segment (start 157.734 95.758) (end 157.734 92.249) (width 0.2) (layer "B.Cu") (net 11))
 (segment (start 154.686 97.028) (end 155.956 95.758) (width 0.2) (layer "B.Cu") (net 11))
 (segment (start 160.782 89.408) (end 158.75 89.408) (width 0.2) (layer "F.Cu") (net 12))
 (via (at 160.782 89.408) (size 1.5) (drill 0.7) (layers "F.Cu" "B.Cu") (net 12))
 (segment (start 160.782 92.456) (end 159.512 93.726) (width 0.2) (layer "B.Cu") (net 12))
 (segment (start 159.512 93.726) (end 158.703 93.726) (width 0.2) (layer "B.Cu") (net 12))
 (segment (start 160.782 89.408) (end 160.782 92.456) (width 0.2) (layer "B.Cu") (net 12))
 (segment (start 154.94 91.948) (end 150.423002 91.948) (width 0.508) (layer "F.Cu") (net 4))
 (segment (start 150.423002 91.948) (end 150.423002 90.424) (width 0.508) (layer "F.Cu") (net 4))
 (segment (start 146.558 91.948) (end 150.423002 91.948) (width 0.508) (layer "F.Cu") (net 4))
 (segment (start 150.423002 91.948) (end 150.423002 90.460998) (width 0.508) (layer "F.Cu") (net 4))
 (segment (start 150.423002 90.460998) (end 150.423002 90.424) (width 0.2) (layer "F.Cu") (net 4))
 (via (at 154.94 91.948) (size 1.5) (drill 0.7) (layers "F.Cu" "B.Cu") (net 4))
 (via (at 146.558 91.948) (size 1.5) (drill 0.7) (layers "F.Cu" "B.Cu") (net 4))
 (segment (start 156.718 93.726) (end 156.878 93.726) (width 0.2) (layer "B.Cu") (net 4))
 (segment (start 146.558 92.202) (end 145.288 93.472) (width 0.2) (layer "B.Cu") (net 4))
 (segment (start 154.94 91.948) (end 156.718 93.726) (width 0.2) (layer "B.Cu") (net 4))
 (segment (start 146.558 91.948) (end 146.558 92.202) (width 0.2) (layer "B.Cu") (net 4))
 (segment (start 145.288 93.472) (end 145.288 93.726) (width 0.2) (layer "B.Cu") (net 4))
 (segment (start 140.97 89.408) (end 142.98 89.408) (width 0.508) (layer "F.Cu") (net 9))
 (via (at 140.97 89.408) (size 1.5) (drill 0.7) (layers "F.Cu" "B.Cu") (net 9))
 (segment (start 140.97 89.408) (end 140.97 92.456) (width 0.2) (layer "B.Cu") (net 9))
 (segment (start 140.97 92.456) (end 142.24 93.726) (width 0.2) (layer "B.Cu") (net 9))
 (segment (start 142.24 93.726) (end 143.463 93.726) (width 0.2) (layer "B.Cu") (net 9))
 (segment (start 156.7815 88.9508) (end 156.4132 88.9508) (width 0.2) (layer "B.Cu") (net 14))
 (segment (start 156.4132 88.9508) (end 153.717 91.647) (width 0.2) (layer "B.Cu") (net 14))
 (segment (start 153.717 91.647) (end 153.717 93.726) (width 0.2) (layer "B.Cu") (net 14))
 (segment (start 157.734 86.868) (end 157.734 89.916) (width 0.2) (layer "B.Cu") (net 13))
 (segment (start 157.734 89.916) (end 158.75 90.932) (width 0.2) (layer "B.Cu") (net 13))
 (segment (start 158.75 90.932) (end 158.75 91.44) (width 0.2) (layer "B.Cu") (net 13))
 (segment (start 144.907 88.011) (end 147.828 90.932) (width 0.2) (layer "B.Cu") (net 15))
 (segment (start 147.828 90.932) (end 147.828 93.726) (width 0.2) (layer "B.Cu") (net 15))
 (segment (start 144.907 87.122) (end 144.907 88.011) (width 0.2) (layer "B.Cu") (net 15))
 (segment (start 142.494 90.424) (end 142.494 91.694) (width 0.2) (layer "B.Cu") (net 16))
 (segment (start 143.764 89.154) (end 142.494 90.424) (width 0.2) (layer "B.Cu") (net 16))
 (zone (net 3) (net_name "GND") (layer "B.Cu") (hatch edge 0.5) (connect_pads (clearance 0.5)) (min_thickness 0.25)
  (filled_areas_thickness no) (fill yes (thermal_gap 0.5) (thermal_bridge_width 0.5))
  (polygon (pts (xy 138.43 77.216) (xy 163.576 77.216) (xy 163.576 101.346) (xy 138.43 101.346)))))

